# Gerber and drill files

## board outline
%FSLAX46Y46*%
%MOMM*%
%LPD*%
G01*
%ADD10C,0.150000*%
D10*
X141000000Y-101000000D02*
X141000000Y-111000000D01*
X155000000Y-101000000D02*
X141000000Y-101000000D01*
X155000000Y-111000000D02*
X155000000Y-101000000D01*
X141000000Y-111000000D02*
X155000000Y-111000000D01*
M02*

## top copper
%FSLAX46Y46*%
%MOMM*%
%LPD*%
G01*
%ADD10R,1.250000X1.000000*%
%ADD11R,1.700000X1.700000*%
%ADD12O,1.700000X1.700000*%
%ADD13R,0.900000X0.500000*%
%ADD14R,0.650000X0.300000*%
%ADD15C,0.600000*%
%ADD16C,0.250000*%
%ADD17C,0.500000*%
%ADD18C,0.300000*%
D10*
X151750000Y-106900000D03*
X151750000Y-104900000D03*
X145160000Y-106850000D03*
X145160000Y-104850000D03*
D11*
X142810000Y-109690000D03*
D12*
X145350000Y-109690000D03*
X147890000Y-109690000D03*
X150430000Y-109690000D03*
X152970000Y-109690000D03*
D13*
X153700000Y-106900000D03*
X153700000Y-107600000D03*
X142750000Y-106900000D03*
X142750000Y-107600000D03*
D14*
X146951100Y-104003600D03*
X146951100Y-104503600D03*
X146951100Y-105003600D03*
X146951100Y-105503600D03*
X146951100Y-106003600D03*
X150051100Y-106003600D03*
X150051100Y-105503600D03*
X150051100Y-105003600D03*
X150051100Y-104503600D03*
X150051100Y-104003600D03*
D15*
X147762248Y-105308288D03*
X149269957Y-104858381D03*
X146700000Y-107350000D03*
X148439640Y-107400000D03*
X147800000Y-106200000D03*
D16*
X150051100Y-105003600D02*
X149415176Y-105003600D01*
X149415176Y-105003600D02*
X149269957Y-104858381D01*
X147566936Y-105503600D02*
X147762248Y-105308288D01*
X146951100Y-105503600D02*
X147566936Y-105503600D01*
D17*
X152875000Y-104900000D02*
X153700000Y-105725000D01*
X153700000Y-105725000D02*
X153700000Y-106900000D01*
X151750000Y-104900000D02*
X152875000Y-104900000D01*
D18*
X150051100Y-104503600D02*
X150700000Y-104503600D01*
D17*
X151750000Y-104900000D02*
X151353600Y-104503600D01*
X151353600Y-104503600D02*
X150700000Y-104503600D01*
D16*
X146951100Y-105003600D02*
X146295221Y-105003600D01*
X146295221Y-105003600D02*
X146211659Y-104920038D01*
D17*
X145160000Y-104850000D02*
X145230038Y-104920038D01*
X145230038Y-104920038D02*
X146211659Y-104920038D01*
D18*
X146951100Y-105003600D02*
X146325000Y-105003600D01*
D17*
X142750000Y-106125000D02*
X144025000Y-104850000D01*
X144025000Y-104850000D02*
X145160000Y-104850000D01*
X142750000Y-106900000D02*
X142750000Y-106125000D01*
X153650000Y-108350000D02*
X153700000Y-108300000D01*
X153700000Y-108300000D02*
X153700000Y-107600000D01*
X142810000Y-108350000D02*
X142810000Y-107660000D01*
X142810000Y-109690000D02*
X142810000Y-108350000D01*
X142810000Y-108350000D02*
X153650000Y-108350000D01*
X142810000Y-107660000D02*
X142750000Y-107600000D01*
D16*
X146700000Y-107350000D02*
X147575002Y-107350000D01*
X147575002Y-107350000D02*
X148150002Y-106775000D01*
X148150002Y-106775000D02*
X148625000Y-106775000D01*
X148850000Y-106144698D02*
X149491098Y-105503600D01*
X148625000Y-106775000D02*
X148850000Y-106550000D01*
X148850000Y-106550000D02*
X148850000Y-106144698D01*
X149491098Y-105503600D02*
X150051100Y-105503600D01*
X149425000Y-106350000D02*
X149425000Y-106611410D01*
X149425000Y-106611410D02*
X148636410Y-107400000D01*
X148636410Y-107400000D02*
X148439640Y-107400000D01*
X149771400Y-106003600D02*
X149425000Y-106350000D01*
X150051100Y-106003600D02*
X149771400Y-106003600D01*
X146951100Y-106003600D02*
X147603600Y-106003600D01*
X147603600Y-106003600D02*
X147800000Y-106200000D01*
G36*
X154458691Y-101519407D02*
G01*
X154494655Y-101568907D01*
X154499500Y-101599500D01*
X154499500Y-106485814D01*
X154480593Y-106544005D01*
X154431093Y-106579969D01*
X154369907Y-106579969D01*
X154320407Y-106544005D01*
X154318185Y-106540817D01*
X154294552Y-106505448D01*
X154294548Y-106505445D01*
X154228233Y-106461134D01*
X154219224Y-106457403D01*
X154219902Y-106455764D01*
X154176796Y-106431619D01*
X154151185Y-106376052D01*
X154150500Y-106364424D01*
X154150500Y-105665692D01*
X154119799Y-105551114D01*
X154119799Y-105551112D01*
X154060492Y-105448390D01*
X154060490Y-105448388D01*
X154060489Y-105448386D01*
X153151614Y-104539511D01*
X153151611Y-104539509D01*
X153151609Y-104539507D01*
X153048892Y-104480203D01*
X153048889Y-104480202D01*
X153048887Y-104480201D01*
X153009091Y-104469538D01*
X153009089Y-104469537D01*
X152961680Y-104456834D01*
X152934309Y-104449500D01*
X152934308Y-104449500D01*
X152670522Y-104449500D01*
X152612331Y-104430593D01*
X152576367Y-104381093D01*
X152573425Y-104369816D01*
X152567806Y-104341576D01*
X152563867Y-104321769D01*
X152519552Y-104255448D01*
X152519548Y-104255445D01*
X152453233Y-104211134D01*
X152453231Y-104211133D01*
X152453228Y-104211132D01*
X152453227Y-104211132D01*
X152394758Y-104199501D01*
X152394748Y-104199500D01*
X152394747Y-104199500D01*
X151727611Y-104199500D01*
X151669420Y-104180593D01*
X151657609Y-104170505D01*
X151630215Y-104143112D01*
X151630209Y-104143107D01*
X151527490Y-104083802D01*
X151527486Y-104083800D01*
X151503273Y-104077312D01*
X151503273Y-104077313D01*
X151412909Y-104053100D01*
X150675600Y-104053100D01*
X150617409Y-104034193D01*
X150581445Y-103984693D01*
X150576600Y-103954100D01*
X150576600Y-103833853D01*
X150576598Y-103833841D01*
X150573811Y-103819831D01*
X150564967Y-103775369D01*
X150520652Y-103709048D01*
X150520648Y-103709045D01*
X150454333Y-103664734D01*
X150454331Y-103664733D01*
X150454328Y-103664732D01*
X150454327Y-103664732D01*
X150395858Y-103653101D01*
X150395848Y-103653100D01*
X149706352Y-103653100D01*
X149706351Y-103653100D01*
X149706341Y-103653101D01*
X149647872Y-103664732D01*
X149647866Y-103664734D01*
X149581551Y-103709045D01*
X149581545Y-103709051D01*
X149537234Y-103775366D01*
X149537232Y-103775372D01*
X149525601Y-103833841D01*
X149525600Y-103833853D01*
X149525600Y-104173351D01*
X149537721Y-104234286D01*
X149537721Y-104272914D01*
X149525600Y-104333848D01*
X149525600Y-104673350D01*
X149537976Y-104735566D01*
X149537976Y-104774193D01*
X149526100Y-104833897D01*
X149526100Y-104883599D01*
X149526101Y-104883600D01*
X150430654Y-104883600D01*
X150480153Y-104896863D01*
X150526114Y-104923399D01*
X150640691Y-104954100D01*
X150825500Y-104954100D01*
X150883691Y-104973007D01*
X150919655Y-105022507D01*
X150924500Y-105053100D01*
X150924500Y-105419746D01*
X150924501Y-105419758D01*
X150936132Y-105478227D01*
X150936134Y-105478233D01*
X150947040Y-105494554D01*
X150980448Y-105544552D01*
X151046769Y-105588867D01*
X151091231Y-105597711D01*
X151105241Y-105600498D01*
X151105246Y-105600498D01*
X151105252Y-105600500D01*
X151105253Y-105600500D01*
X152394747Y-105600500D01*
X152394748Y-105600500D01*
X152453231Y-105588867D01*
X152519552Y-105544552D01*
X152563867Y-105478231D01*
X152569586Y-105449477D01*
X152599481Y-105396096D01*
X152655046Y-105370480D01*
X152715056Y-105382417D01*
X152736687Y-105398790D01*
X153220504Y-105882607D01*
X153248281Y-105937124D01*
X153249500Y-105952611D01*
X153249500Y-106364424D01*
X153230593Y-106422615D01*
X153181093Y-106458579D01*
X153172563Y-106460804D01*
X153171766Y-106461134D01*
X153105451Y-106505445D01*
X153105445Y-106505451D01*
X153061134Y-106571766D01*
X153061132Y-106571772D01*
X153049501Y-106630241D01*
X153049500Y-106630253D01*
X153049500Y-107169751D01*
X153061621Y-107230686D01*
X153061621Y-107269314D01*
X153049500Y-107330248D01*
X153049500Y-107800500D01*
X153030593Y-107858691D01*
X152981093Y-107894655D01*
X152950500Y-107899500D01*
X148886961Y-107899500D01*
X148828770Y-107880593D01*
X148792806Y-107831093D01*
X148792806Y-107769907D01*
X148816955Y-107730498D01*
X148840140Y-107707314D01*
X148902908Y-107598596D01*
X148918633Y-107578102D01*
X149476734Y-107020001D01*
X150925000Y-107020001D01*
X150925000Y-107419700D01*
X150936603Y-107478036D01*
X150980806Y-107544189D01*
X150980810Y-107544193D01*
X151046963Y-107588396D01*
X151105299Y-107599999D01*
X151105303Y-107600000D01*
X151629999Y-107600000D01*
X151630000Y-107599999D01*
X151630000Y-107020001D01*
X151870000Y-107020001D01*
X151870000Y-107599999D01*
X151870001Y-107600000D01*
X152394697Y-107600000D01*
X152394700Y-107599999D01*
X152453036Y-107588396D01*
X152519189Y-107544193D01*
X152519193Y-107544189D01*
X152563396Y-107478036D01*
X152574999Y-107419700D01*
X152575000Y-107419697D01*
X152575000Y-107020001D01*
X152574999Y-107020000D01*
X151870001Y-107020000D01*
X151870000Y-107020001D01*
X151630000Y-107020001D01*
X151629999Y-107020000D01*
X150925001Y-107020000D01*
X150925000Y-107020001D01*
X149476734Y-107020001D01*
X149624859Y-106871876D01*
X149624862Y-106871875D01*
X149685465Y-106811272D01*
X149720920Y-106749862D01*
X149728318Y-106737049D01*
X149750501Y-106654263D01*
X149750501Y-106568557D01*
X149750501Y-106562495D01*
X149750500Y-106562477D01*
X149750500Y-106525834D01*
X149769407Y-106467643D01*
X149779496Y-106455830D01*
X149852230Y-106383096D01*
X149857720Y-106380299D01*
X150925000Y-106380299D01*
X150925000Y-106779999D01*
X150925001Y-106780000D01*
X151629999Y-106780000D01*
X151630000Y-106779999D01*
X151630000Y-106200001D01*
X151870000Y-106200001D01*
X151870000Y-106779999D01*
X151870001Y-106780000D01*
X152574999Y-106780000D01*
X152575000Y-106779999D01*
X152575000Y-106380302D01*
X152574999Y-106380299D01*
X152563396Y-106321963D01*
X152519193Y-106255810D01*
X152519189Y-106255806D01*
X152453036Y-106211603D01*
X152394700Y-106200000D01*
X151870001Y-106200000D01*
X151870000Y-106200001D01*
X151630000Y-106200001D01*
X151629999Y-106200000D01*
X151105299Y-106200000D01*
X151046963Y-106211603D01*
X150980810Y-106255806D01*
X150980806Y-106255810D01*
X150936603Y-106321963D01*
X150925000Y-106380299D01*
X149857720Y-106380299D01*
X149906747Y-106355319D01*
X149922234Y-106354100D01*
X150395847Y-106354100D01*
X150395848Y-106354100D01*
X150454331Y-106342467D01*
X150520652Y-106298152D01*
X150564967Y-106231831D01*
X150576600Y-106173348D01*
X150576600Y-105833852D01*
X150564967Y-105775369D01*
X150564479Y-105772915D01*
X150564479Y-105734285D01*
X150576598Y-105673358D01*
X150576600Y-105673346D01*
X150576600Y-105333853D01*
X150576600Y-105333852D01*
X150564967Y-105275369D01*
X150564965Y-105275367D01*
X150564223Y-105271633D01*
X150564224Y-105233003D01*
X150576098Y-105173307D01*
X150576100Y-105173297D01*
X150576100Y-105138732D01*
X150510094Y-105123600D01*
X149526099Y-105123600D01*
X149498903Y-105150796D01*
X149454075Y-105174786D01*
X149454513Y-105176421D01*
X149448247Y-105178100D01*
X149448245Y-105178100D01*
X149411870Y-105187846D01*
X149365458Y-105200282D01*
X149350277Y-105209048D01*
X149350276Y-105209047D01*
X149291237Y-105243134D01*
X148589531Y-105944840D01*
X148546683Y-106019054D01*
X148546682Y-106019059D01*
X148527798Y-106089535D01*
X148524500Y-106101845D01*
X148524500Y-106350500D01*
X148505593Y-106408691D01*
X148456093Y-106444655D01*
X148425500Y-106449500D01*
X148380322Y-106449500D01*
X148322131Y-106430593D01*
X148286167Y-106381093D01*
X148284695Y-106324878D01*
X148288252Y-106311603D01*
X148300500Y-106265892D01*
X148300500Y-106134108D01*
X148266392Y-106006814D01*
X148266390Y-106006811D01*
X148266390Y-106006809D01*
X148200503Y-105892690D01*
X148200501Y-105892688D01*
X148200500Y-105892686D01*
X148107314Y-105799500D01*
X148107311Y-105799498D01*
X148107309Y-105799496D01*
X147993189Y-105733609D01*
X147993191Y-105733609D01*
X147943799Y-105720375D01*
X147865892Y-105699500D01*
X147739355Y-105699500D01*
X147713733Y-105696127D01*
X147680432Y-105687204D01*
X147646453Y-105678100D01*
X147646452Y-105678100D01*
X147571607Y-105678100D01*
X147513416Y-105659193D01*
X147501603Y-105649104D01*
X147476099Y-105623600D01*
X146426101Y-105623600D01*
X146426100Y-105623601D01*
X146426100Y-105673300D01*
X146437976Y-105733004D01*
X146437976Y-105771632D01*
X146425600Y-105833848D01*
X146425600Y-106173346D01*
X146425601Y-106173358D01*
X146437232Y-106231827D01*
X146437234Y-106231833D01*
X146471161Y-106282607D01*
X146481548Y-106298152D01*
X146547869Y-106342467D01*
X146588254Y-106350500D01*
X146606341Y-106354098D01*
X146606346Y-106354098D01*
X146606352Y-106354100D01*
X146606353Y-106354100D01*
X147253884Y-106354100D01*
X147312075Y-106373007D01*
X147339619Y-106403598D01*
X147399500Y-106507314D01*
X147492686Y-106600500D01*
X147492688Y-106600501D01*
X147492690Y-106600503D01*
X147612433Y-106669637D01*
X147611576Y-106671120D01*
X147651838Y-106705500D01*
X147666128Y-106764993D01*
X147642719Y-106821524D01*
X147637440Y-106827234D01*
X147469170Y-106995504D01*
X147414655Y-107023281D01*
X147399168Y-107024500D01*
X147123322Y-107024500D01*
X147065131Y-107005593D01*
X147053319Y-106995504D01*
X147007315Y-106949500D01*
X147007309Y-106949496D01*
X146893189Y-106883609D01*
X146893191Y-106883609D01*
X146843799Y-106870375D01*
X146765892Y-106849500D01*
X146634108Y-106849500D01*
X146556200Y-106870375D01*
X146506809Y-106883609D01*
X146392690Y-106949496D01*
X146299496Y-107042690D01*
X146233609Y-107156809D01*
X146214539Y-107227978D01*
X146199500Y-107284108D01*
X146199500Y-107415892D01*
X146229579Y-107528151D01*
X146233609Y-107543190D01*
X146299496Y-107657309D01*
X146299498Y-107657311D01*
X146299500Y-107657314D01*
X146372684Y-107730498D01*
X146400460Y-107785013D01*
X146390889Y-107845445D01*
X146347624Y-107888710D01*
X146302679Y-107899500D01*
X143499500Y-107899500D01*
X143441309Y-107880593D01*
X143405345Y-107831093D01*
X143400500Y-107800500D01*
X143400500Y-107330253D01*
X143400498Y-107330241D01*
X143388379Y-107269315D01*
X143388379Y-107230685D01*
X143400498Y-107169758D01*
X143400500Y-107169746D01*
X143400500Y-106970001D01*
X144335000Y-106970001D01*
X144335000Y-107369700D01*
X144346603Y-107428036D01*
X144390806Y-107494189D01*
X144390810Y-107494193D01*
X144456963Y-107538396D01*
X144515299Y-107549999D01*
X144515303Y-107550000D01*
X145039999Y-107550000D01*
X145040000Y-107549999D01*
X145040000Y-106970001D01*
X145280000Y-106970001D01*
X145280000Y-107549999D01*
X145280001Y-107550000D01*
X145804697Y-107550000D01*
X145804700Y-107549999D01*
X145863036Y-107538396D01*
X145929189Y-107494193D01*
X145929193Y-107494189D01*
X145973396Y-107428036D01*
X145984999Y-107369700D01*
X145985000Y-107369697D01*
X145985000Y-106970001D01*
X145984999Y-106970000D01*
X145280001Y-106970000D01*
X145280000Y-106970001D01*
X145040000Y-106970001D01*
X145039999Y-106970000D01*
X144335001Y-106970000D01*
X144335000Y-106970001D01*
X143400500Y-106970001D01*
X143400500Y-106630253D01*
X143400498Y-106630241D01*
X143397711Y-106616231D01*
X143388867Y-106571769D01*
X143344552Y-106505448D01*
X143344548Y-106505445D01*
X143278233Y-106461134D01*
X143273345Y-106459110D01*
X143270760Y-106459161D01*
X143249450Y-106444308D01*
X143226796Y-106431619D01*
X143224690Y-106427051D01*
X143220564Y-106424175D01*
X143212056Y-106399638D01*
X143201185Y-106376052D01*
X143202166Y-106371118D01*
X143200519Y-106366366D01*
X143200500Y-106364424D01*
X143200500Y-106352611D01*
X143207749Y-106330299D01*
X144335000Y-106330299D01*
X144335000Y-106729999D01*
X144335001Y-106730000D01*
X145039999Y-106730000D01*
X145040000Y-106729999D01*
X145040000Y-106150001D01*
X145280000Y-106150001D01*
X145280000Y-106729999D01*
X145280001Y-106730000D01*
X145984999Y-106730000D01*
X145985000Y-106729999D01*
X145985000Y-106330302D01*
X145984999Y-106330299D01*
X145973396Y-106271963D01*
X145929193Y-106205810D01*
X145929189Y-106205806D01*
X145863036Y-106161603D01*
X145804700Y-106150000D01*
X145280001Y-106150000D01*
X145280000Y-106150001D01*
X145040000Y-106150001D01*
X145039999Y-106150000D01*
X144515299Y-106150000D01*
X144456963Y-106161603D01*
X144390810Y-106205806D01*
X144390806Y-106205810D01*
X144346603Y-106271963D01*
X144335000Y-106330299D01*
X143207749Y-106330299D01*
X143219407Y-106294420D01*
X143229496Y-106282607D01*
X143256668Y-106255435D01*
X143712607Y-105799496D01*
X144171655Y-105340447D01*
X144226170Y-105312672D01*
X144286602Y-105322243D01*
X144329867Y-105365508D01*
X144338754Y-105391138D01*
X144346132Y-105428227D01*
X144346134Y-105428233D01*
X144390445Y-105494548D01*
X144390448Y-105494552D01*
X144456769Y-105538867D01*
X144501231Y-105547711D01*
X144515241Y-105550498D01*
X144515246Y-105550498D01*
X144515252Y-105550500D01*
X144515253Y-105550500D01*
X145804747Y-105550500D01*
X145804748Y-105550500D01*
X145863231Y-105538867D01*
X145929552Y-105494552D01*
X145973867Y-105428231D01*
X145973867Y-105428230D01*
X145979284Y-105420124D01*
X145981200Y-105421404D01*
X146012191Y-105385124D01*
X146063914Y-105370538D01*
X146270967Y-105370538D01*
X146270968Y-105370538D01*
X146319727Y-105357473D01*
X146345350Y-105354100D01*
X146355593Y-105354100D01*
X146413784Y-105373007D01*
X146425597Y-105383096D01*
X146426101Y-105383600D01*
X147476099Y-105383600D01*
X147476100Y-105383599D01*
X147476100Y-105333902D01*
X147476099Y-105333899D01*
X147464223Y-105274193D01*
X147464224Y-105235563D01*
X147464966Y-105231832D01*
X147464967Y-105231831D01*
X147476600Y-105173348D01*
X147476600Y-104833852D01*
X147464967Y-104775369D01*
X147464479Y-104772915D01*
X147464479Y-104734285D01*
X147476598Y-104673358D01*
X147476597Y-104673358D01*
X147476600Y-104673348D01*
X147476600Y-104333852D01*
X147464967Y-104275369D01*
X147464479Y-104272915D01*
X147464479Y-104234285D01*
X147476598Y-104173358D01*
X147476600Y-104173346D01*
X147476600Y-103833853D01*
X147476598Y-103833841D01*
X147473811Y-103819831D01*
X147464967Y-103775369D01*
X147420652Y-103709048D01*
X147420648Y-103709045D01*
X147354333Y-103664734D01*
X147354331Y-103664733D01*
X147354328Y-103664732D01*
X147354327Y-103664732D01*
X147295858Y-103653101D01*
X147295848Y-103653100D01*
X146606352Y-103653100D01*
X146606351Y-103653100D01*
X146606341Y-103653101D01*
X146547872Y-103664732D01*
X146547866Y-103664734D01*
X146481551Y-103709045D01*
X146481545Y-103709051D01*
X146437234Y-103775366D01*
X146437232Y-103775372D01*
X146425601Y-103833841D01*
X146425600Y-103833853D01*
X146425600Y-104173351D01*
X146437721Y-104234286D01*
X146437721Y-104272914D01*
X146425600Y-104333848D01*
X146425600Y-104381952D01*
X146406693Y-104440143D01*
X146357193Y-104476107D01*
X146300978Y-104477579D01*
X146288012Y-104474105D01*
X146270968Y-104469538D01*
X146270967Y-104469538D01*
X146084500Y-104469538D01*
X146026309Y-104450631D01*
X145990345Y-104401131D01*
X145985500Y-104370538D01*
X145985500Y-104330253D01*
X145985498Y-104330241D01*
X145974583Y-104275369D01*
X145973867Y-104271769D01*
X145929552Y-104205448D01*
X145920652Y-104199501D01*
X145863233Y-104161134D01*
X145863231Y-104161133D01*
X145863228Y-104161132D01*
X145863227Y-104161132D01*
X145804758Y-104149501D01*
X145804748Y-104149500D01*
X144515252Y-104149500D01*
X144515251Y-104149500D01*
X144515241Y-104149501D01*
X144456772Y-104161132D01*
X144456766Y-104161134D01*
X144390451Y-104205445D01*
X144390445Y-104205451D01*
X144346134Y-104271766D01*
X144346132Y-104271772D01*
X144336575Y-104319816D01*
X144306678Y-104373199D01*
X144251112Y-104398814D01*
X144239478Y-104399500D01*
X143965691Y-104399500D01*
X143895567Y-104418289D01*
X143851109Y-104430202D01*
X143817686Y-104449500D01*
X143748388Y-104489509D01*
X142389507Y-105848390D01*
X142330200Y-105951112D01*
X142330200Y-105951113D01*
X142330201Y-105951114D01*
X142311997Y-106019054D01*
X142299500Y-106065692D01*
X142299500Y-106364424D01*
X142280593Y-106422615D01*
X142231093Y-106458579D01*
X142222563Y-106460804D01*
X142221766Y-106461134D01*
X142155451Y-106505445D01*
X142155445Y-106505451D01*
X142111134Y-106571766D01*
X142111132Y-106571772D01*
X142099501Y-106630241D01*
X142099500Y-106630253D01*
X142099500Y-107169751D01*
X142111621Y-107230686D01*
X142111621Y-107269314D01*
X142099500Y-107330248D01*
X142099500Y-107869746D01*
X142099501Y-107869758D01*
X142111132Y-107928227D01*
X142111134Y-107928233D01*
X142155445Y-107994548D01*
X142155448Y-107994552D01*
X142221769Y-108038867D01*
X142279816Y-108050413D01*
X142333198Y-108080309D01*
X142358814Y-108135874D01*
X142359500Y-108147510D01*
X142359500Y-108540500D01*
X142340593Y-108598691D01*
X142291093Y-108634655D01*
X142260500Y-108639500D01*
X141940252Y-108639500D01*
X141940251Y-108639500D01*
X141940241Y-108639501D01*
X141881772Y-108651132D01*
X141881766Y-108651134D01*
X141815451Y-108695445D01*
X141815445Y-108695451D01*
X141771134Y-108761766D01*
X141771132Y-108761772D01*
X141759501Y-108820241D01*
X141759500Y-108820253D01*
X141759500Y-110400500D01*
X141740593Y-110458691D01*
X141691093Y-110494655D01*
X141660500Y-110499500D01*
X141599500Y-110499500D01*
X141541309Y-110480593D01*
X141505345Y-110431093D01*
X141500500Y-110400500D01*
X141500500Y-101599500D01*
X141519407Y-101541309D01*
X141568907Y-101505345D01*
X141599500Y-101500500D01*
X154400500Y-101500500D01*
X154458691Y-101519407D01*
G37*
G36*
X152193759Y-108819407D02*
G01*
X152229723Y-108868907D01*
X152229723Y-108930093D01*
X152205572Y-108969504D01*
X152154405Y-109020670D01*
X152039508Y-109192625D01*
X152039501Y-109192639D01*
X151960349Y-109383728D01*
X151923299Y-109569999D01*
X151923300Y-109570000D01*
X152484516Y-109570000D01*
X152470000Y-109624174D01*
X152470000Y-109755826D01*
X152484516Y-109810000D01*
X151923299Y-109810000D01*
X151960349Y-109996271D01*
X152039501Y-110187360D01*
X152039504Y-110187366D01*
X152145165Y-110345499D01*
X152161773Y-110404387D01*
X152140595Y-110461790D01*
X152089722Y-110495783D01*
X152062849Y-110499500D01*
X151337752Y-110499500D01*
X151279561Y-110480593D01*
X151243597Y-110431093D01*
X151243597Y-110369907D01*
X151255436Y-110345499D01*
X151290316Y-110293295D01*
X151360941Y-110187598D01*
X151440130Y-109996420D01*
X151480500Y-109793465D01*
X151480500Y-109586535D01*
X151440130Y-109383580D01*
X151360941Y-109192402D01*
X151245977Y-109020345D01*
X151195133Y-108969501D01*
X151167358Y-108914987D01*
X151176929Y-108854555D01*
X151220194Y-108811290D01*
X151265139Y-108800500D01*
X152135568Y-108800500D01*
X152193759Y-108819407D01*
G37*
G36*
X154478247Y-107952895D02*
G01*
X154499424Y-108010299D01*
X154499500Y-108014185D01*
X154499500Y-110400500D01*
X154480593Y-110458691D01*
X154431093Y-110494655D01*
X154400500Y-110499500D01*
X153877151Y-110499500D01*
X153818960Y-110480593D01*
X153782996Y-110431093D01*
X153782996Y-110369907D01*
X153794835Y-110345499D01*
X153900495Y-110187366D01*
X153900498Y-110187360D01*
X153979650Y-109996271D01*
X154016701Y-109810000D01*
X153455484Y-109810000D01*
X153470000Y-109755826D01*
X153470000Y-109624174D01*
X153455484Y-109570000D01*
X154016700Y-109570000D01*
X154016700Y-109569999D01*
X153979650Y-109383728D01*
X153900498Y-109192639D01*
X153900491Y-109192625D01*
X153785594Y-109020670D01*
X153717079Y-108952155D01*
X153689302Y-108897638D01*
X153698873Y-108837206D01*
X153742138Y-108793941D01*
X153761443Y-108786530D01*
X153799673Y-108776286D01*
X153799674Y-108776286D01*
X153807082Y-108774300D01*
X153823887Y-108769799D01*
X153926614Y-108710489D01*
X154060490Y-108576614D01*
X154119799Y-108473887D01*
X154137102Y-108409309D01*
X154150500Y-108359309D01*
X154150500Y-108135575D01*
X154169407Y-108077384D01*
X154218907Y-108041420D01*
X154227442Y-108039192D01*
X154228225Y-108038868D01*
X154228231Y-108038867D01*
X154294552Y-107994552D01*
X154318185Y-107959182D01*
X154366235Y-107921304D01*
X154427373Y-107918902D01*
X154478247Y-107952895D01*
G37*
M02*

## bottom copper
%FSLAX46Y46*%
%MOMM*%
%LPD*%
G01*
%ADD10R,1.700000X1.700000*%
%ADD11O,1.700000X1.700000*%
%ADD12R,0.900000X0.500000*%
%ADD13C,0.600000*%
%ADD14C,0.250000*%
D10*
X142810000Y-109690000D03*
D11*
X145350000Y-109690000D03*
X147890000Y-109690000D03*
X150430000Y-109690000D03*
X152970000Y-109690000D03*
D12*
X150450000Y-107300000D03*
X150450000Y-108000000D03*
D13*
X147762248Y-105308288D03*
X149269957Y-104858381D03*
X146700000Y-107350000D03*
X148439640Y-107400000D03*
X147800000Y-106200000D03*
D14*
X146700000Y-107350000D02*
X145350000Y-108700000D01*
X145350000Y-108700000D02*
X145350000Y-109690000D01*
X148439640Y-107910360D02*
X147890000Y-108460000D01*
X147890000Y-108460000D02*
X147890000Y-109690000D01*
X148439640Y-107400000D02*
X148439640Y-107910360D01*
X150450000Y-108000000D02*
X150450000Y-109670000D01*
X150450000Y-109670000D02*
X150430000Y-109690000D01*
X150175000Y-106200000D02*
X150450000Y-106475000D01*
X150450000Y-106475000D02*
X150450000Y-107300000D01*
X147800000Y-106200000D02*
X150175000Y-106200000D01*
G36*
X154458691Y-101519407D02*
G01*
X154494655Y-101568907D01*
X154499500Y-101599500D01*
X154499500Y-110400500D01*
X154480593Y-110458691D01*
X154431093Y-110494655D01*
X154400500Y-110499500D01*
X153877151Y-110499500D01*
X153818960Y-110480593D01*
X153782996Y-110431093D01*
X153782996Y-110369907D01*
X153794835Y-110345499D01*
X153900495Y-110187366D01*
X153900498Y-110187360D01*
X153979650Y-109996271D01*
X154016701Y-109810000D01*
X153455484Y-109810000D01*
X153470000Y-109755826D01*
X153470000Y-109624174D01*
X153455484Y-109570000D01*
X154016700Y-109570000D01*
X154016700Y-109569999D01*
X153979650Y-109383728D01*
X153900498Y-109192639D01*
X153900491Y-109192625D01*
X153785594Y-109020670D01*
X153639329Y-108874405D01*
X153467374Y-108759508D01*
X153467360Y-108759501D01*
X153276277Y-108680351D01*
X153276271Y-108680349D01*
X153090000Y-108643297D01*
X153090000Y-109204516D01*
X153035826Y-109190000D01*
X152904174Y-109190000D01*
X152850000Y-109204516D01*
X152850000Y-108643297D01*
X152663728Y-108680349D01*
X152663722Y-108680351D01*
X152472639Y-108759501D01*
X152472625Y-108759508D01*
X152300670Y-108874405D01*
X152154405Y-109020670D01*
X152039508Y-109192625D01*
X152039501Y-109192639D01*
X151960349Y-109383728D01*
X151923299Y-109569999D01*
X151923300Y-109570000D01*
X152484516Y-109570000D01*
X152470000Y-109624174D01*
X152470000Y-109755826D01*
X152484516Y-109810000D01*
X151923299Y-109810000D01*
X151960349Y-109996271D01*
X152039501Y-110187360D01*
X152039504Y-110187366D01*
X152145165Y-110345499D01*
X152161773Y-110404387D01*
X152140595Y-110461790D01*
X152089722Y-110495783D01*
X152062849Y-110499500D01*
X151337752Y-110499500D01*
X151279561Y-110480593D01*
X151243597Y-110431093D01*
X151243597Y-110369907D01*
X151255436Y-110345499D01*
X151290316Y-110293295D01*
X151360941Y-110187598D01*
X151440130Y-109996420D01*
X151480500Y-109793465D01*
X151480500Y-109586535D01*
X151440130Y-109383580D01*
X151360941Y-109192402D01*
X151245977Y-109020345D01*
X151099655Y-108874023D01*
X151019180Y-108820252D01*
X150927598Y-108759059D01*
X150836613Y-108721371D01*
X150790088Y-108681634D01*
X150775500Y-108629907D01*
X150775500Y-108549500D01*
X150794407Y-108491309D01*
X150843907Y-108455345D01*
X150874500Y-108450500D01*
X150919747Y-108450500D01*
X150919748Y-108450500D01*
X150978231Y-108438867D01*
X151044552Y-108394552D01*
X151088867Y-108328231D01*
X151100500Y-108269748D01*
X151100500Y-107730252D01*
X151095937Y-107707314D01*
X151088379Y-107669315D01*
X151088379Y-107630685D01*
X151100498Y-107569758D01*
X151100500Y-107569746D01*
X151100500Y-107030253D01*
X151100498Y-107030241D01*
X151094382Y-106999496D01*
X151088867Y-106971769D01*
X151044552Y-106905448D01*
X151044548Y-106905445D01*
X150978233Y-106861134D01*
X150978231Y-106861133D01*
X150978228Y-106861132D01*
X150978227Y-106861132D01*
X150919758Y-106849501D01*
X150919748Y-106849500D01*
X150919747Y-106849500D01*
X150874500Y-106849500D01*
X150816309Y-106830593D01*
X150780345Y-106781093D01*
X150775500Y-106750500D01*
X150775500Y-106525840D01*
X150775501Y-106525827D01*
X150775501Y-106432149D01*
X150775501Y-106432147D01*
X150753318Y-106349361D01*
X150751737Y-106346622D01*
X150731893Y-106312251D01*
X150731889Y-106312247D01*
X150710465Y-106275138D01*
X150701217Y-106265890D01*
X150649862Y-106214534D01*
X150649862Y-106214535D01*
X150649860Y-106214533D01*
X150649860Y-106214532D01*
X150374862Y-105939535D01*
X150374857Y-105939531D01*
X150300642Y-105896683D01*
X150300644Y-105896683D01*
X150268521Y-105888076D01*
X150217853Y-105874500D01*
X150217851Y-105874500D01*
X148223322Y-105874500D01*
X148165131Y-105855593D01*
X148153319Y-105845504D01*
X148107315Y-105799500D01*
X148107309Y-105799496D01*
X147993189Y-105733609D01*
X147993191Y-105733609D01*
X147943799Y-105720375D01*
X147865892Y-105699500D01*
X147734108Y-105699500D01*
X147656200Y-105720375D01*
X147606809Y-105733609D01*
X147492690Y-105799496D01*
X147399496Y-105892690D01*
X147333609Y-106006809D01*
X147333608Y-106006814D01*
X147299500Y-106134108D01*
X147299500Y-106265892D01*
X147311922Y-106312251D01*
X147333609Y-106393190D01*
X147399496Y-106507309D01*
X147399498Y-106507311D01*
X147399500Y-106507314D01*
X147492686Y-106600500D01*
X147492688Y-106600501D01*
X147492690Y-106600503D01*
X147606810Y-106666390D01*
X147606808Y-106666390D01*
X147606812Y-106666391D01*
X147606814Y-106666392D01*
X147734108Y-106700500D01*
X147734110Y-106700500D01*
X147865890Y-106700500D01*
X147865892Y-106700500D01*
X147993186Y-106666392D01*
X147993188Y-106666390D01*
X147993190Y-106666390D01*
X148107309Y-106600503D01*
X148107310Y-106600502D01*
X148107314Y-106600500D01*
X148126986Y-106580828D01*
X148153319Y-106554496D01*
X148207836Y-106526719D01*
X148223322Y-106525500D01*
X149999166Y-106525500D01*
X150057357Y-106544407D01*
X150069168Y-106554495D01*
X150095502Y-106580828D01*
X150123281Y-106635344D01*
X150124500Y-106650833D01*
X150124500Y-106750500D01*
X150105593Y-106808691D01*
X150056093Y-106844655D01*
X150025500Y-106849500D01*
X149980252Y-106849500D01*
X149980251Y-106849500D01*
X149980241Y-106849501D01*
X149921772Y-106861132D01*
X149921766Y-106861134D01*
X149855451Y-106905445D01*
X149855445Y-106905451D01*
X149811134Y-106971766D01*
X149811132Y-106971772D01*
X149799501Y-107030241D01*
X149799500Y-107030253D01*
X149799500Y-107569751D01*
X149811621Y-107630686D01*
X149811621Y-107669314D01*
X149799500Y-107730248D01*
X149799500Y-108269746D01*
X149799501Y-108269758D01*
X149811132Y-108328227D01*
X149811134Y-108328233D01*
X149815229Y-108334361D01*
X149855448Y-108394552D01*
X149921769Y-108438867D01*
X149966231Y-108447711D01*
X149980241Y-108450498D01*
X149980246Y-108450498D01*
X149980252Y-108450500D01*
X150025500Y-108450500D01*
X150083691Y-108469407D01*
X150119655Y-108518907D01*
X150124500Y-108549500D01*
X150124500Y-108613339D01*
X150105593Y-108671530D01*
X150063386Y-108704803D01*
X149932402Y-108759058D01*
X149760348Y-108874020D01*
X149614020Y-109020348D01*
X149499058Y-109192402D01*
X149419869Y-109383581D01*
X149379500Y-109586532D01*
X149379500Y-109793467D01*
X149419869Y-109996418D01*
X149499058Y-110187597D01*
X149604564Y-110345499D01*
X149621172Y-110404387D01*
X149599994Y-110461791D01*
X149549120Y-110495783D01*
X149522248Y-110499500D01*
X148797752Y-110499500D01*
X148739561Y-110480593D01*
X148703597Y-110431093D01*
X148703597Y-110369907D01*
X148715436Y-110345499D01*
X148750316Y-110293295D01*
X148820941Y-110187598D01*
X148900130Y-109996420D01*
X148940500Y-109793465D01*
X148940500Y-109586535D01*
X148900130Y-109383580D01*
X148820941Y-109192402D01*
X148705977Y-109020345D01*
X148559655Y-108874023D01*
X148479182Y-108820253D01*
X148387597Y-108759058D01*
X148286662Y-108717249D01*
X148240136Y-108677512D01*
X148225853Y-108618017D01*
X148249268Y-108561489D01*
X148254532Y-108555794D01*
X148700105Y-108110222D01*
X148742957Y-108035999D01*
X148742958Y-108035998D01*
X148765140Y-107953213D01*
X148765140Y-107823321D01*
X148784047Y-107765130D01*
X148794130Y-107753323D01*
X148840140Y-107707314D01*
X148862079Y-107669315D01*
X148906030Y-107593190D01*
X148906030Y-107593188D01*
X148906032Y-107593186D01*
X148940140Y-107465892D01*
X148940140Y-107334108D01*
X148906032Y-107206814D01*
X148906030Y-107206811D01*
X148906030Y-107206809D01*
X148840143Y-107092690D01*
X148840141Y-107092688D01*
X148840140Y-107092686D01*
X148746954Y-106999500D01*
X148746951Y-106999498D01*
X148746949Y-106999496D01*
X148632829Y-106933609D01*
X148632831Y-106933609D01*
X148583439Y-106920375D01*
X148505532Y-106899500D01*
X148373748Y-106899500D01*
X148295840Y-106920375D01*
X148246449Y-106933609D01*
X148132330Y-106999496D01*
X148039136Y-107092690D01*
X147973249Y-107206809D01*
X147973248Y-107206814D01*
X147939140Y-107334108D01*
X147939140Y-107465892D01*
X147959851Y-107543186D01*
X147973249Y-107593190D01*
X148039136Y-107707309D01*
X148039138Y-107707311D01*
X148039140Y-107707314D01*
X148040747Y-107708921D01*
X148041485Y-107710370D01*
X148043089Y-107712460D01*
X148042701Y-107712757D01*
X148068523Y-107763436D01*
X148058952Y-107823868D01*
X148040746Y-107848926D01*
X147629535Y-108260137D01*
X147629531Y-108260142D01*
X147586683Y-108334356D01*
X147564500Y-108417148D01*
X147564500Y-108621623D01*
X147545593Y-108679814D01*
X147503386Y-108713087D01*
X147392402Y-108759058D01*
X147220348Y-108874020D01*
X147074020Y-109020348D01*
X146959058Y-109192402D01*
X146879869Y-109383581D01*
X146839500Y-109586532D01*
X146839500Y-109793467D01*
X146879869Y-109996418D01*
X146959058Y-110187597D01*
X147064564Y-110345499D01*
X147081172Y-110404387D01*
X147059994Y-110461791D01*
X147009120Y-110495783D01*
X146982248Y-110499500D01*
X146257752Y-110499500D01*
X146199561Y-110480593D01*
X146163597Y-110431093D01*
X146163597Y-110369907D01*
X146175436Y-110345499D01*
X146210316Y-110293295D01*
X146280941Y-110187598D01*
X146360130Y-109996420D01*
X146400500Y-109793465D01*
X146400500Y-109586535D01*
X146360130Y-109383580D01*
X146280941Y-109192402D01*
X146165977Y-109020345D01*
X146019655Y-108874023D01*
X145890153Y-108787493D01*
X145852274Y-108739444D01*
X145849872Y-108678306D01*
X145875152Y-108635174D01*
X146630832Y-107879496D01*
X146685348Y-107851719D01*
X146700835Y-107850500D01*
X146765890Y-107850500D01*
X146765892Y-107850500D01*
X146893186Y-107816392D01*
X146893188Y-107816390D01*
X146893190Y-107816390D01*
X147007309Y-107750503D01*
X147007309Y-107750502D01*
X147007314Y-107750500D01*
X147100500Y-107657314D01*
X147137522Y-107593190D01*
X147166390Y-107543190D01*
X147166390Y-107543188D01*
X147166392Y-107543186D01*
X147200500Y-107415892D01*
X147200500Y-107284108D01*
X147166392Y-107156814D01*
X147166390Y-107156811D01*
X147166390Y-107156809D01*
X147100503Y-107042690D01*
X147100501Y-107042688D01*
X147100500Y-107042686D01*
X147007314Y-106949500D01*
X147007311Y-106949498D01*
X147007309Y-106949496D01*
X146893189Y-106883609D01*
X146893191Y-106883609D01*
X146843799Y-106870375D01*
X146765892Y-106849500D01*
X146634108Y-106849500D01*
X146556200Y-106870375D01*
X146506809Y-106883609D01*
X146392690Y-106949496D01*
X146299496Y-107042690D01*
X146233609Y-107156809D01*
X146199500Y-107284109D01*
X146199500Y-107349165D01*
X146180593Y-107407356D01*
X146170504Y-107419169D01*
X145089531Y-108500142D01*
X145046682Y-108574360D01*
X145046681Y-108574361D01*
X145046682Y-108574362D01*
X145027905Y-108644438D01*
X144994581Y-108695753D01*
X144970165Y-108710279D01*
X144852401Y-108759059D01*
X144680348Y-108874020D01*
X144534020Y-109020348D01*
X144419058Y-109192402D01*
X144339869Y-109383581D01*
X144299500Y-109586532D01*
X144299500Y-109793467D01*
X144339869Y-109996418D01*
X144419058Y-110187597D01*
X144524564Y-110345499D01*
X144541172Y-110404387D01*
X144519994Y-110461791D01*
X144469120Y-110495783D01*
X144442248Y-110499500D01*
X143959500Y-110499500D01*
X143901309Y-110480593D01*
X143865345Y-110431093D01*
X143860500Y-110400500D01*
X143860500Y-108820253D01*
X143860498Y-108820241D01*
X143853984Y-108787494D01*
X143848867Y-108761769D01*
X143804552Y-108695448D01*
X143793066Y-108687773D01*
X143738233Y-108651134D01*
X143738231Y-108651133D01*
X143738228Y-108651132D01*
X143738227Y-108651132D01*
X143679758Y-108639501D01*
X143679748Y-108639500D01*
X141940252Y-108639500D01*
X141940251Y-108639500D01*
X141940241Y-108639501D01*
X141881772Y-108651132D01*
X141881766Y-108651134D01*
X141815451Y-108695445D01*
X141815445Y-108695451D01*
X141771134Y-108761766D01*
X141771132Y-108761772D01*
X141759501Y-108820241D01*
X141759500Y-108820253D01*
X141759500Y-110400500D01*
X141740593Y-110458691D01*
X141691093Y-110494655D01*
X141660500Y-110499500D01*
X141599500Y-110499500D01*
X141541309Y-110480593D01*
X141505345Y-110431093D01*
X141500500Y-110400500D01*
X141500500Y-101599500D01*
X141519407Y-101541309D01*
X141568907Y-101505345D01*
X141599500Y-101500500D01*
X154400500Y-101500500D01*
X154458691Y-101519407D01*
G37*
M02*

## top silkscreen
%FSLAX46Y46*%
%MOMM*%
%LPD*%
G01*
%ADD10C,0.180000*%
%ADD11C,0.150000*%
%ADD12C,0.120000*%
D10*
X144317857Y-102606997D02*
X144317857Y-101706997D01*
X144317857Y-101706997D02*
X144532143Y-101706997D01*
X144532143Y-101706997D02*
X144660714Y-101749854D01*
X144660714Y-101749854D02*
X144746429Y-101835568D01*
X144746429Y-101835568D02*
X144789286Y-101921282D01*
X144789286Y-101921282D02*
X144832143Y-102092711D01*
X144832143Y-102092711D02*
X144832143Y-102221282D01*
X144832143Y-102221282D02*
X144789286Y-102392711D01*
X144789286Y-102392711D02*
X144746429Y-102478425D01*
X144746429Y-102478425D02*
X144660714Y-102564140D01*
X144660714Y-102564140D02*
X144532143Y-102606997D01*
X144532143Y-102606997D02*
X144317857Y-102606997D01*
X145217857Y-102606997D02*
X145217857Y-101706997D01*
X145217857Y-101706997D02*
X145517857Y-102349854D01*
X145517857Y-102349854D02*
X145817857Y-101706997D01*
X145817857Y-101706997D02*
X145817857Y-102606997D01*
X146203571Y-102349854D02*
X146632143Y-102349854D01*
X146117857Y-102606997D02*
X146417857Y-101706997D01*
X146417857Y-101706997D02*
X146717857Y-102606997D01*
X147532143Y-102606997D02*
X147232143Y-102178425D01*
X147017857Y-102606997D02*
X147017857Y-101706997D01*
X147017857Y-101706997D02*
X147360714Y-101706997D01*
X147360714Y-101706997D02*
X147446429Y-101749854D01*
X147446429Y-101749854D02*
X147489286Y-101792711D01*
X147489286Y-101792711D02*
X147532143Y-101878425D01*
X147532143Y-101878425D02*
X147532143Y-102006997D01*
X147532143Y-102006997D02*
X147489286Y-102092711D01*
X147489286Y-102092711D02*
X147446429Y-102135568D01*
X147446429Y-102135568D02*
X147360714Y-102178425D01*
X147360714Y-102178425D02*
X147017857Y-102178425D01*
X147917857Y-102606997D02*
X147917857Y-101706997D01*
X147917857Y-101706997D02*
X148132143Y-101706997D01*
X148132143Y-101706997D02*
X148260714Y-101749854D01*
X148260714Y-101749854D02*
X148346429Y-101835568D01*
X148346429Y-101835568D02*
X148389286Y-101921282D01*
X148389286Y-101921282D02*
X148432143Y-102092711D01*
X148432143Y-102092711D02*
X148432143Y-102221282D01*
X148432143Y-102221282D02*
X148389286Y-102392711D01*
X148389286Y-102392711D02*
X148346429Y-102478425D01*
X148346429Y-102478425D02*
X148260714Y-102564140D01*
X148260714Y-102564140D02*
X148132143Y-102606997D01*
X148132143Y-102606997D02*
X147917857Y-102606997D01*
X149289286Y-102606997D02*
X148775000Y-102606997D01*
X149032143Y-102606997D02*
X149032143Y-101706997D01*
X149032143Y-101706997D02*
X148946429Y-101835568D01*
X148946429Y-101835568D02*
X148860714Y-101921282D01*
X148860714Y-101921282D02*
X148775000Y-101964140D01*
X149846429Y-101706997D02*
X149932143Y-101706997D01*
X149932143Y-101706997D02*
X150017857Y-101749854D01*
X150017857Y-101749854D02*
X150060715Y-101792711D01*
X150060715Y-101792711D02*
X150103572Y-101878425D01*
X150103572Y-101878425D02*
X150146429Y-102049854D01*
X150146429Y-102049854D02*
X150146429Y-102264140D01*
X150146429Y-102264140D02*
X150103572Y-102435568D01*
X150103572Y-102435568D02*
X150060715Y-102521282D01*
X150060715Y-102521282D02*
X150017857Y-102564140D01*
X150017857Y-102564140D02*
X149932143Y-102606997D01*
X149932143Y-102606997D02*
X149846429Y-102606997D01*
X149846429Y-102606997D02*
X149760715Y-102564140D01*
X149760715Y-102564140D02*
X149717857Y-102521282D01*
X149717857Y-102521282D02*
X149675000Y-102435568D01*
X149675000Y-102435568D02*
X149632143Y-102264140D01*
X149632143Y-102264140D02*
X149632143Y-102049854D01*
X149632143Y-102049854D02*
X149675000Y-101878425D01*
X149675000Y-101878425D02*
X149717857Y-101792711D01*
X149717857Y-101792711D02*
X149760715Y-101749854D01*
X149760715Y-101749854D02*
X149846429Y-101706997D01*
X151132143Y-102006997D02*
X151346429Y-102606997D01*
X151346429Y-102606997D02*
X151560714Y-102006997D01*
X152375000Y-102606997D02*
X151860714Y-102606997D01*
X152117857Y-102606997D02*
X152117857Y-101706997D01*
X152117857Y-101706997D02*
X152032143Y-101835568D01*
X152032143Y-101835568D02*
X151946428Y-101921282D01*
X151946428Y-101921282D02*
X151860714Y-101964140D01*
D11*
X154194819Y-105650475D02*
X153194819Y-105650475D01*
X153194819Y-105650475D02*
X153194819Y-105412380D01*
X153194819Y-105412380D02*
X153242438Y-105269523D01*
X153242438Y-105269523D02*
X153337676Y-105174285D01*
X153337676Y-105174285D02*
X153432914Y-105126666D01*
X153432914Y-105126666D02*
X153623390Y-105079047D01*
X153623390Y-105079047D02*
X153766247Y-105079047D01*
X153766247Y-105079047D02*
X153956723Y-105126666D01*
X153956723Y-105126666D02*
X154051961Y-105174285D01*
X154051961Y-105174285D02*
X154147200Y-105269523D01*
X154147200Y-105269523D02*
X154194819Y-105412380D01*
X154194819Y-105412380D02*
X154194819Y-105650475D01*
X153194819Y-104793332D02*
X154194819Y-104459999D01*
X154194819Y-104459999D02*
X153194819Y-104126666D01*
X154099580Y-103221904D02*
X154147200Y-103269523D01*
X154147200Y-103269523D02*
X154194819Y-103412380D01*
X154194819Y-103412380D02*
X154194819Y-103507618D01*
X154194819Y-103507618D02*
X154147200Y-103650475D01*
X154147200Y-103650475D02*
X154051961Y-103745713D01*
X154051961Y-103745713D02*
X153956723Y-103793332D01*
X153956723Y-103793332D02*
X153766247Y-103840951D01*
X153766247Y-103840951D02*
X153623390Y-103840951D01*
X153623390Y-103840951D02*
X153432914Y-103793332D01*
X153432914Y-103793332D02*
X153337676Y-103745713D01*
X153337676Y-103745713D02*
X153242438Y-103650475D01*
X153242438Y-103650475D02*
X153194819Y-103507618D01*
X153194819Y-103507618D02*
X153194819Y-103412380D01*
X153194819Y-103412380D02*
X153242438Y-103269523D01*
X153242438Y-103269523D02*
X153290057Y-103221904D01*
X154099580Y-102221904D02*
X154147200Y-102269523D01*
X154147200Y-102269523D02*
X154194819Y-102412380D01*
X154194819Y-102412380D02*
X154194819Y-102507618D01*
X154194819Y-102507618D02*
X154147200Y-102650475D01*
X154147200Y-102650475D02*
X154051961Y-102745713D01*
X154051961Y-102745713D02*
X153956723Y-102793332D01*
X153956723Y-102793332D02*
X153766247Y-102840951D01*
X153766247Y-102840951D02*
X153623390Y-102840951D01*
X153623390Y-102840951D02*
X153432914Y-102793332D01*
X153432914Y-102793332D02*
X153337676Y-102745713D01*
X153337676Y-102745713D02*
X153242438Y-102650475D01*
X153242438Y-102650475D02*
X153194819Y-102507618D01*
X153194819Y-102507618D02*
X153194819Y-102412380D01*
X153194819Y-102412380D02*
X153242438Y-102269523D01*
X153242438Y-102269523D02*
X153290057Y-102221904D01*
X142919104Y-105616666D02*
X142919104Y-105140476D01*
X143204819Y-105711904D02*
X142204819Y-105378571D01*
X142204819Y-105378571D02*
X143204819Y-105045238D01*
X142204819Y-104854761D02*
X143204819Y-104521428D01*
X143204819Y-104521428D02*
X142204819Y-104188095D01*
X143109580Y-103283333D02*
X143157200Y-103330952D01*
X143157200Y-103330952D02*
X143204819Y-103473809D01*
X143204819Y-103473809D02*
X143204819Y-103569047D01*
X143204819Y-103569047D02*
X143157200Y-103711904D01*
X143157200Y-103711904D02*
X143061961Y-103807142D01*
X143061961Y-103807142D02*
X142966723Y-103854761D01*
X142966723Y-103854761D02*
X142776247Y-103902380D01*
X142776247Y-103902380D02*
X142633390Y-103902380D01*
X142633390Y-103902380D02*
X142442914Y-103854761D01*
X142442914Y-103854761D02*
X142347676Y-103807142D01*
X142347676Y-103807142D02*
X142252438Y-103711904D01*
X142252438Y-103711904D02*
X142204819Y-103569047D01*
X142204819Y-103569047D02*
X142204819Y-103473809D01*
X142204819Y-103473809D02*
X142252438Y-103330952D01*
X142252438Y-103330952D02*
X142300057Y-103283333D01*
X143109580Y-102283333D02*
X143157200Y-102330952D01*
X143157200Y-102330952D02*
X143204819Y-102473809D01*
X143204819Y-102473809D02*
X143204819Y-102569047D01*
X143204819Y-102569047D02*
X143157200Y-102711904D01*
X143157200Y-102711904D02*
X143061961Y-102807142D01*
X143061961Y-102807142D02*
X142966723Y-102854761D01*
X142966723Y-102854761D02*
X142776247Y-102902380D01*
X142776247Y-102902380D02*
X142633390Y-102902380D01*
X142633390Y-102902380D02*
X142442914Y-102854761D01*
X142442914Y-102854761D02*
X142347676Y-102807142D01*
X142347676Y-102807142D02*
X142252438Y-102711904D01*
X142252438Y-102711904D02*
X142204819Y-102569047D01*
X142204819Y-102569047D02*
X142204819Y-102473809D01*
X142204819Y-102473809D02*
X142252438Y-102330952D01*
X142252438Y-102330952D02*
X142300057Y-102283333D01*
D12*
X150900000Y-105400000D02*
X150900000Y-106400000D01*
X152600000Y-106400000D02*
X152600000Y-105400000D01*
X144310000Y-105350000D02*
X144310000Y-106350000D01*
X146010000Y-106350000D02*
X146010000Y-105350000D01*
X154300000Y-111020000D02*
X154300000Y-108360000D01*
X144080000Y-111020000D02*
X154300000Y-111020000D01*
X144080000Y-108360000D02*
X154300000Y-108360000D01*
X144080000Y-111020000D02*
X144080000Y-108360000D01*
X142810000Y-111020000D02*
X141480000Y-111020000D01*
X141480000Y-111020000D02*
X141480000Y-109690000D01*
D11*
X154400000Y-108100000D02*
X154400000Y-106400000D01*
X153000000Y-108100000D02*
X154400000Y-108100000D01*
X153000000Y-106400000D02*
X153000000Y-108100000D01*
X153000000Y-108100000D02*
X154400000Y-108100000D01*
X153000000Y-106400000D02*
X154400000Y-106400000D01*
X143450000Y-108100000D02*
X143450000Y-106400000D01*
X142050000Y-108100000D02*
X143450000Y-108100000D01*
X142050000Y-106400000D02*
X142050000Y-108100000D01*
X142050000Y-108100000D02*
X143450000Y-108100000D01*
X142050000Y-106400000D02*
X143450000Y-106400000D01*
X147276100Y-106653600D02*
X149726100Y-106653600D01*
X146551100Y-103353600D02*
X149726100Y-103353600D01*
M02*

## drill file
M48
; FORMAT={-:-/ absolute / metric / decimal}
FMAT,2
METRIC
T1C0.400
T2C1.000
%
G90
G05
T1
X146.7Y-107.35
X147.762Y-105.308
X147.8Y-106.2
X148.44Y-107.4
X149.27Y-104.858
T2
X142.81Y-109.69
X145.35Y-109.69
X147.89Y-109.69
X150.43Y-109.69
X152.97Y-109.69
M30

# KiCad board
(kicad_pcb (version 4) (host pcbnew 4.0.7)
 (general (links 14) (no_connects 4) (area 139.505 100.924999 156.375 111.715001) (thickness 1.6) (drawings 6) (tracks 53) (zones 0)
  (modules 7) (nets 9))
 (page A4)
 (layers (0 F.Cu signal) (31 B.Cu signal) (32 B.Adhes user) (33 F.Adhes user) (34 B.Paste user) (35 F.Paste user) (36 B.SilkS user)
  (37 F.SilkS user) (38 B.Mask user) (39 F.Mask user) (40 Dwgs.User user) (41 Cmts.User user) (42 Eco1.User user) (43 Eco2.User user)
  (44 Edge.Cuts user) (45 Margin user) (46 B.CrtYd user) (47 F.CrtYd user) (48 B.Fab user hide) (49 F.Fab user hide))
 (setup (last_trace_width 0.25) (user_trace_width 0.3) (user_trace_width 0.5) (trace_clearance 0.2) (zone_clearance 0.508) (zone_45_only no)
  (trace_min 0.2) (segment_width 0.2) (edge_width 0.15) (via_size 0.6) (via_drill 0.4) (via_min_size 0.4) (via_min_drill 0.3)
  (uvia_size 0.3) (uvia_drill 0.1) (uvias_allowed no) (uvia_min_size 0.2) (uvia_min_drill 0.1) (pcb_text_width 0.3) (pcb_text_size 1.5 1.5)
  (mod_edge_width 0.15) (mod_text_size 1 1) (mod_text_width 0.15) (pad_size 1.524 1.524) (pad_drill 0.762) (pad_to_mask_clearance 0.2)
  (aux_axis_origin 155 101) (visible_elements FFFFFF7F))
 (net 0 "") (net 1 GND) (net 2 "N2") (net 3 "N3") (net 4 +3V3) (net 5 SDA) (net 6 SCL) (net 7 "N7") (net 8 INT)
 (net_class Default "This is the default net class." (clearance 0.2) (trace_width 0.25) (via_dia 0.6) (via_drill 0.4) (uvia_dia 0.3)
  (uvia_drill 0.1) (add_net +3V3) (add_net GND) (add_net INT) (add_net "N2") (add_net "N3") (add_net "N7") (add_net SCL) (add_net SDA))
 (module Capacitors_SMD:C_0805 (layer F.Cu) (at 151.75 105.9 90)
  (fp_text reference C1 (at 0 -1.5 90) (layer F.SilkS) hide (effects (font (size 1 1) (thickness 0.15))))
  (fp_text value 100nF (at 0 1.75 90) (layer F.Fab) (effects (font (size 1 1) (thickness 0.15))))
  (fp_line (start 0.5 -0.85) (end -0.5 -0.85) (layer F.SilkS) (width 0.12))
  (fp_line (start -0.5 0.85) (end 0.5 0.85) (layer F.SilkS) (width 0.12))
  (pad 1 smd rect (at -1 0 90) (size 1 1.25) (layers F.Cu F.Paste F.Mask) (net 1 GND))
  (pad 2 smd rect (at 1 0 90) (size 1 1.25) (layers F.Cu F.Paste F.Mask) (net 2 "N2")))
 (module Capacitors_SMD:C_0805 (layer F.Cu) (at 145.16 105.85 90)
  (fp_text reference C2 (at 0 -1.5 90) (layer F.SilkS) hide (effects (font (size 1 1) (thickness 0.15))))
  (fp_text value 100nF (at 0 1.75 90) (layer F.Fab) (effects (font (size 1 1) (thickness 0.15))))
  (fp_line (start 0.5 -0.85) (end -0.5 -0.85) (layer F.SilkS) (width 0.12))
  (fp_line (start -0.5 0.85) (end 0.5 0.85) (layer F.SilkS) (width 0.12))
  (pad 1 smd rect (at -1 0 90) (size 1 1.25) (layers F.Cu F.Paste F.Mask) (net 1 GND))
  (pad 2 smd rect (at 1 0 90) (size 1 1.25) (layers F.Cu F.Paste F.Mask) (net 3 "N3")))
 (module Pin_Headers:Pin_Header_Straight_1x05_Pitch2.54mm (layer F.Cu) (at 142.81 109.69 90)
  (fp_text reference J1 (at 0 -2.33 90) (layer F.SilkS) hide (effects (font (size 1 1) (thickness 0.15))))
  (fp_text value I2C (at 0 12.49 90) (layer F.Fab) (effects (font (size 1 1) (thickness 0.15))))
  (fp_line (start -1.33 11.49) (end 1.33 11.49) (layer F.SilkS) (width 0.12))
  (fp_line (start -1.33 1.27) (end -1.33 11.49) (layer F.SilkS) (width 0.12))
  (fp_line (start 1.33 1.27) (end 1.33 11.49) (layer F.SilkS) (width 0.12))
  (fp_line (start -1.33 1.27) (end 1.33 1.27) (layer F.SilkS) (width 0.12))
  (fp_line (start -1.33 0) (end -1.33 -1.33) (layer F.SilkS) (width 0.12))
  (fp_line (start -1.33 -1.33) (end 0 -1.33) (layer F.SilkS) (width 0.12))
  (pad 1 thru_hole rect (at 0 0 90) (size 1.7 1.7) (drill 1) (layers *.Cu *.Mask) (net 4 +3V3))
  (pad 2 thru_hole oval (at 0 2.54 90) (size 1.7 1.7) (drill 1) (layers *.Cu *.Mask) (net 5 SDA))
  (pad 3 thru_hole oval (at 0 5.08 90) (size 1.7 1.7) (drill 1) (layers *.Cu *.Mask) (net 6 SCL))
  (pad 4 thru_hole oval (at 0 7.62 90) (size 1.7 1.7) (drill 1) (layers *.Cu *.Mask) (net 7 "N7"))
  (pad 5 thru_hole oval (at 0 10.16 90) (size 1.7 1.7) (drill 1) (layers *.Cu *.Mask) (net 1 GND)))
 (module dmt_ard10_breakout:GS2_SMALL (layer F.Cu) (at 153.7 107.6)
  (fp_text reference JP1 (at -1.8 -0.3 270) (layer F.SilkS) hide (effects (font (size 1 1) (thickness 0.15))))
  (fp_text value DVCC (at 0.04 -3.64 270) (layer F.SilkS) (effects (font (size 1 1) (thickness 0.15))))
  (fp_line (start 0.7 0.5) (end 0.7 -1.2) (layer F.SilkS) (width 0.15))
  (fp_line (start -0.7 0.5) (end 0.7 0.5) (layer F.SilkS) (width 0.15))
  (fp_line (start -0.7 -1.2) (end -0.7 0.5) (layer F.SilkS) (width 0.15))
  (fp_line (start -0.7 0.5) (end 0.7 0.5) (layer F.SilkS) (width 0.15))
  (fp_line (start -0.7 -1.2) (end 0.7 -1.2) (layer F.SilkS) (width 0.15))
  (pad 1 smd rect (at 0 -0.7) (size 0.9 0.5) (layers F.Cu F.Paste F.Mask) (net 2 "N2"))
  (pad 2 smd rect (at 0 0) (size 0.9 0.5) (layers F.Cu F.Paste F.Mask) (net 4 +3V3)))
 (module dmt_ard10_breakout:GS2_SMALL (layer B.Cu) (at 150.45 108 180)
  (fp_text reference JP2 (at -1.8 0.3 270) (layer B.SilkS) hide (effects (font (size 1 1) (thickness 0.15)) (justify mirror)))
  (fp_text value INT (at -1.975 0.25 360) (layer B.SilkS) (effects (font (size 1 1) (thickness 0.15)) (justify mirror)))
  (pad 1 smd rect (at 0 0.7 180) (size 0.9 0.5) (layers B.Cu B.Paste B.Mask) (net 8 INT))
  (pad 2 smd rect (at 0 0 180) (size 0.9 0.5) (layers B.Cu B.Paste B.Mask) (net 7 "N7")))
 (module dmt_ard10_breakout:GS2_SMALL (layer F.Cu) (at 142.75 107.6)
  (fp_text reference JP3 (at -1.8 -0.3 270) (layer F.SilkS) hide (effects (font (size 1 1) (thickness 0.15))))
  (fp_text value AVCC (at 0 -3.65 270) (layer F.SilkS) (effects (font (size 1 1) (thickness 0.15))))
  (fp_line (start 0.7 0.5) (end 0.7 -1.2) (layer F.SilkS) (width 0.15))
  (fp_line (start -0.7 0.5) (end 0.7 0.5) (layer F.SilkS) (width 0.15))
  (fp_line (start -0.7 -1.2) (end -0.7 0.5) (layer F.SilkS) (width 0.15))
  (fp_line (start -0.7 0.5) (end 0.7 0.5) (layer F.SilkS) (width 0.15))
  (fp_line (start -0.7 -1.2) (end 0.7 -1.2) (layer F.SilkS) (width 0.15))
  (pad 1 smd rect (at 0 -0.7) (size 0.9 0.5) (layers F.Cu F.Paste F.Mask) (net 3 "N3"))
  (pad 2 smd rect (at 0 0) (size 0.9 0.5) (layers F.Cu F.Paste F.Mask) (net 4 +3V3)))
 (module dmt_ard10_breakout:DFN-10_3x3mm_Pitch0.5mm (layer F.Cu) (at 148.5011 105.0036)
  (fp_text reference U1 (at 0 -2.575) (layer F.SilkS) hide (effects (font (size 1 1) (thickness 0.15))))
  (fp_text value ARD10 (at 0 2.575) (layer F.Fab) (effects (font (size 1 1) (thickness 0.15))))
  (fp_line (start -1.225 1.65) (end 1.225 1.65) (layer F.SilkS) (width 0.15))
  (fp_line (start -1.95 -1.65) (end 1.225 -1.65) (layer F.SilkS) (width 0.15))
  (pad 1 smd rect (at -1.55 -1) (size 0.65 0.3) (layers F.Cu F.Paste F.Mask))
  (pad 2 smd rect (at -1.55 -0.5) (size 0.65 0.3) (layers F.Cu F.Paste F.Mask))
  (pad 3 smd rect (at -1.55 0) (size 0.65 0.3) (layers F.Cu F.Paste F.Mask) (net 3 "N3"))
  (pad 4 smd rect (at -1.55 0.5) (size 0.65 0.3) (layers F.Cu F.Paste F.Mask) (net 1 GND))
  (pad 5 smd rect (at -1.55 1) (size 0.65 0.3) (layers F.Cu F.Paste F.Mask) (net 8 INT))
  (pad 6 smd rect (at 1.55 1) (size 0.65 0.3) (layers F.Cu F.Paste F.Mask) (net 6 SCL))
  (pad 7 smd rect (at 1.55 0.5) (size 0.65 0.3) (layers F.Cu F.Paste F.Mask) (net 5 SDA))
  (pad 8 smd rect (at 1.55 0) (size 0.65 0.3) (layers F.Cu F.Paste F.Mask) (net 1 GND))
  (pad 9 smd rect (at 1.55 -0.5) (size 0.65 0.3) (layers F.Cu F.Paste F.Mask) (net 2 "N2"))
  (pad 10 smd rect (at 1.55 -1) (size 0.65 0.3) (layers F.Cu F.Paste F.Mask)))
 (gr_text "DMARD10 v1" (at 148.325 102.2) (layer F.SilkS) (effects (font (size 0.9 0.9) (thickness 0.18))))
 (gr_line (start 141 101) (end 141 111) (layer Edge.Cuts) (width 0.15))
 (gr_line (start 155 101) (end 141 101) (layer Edge.Cuts) (width 0.15))
 (gr_line (start 155 111) (end 155 101) (layer Edge.Cuts) (width 0.15))
 (gr_line (start 141 111) (end 155 111) (layer Edge.Cuts) (width 0.15))
 (segment (start 150.0511 105.0036) (end 149.415176 105.0036) (width 0.25) (layer F.Cu) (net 1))
 (segment (start 149.415176 105.0036) (end 149.269957 104.858381) (width 0.25) (layer F.Cu) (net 1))
 (segment (start 147.566936 105.5036) (end 147.762248 105.308288) (width 0.25) (layer F.Cu) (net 1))
 (segment (start 146.9511 105.5036) (end 147.566936 105.5036) (width 0.25) (layer F.Cu) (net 1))
 (via (at 147.762248 105.308288) (size 0.6) (drill 0.4) (layers F.Cu B.Cu) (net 1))
 (via (at 149.269957 104.858381) (size 0.6) (drill 0.4) (layers F.Cu B.Cu) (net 1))
 (segment (start 152.875 104.9) (end 153.7 105.725) (width 0.5) (layer F.Cu) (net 2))
 (segment (start 153.7 105.725) (end 153.7 106.9) (width 0.5) (layer F.Cu) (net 2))
 (segment (start 151.75 104.9) (end 152.875 104.9) (width 0.5) (layer F.Cu) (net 2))
 (segment (start 150.0511 104.5036) (end 150.7 104.5036) (width 0.3) (layer F.Cu) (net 2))
 (segment (start 151.75 104.9) (end 151.3536 104.5036) (width 0.5) (layer F.Cu) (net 2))
 (segment (start 151.3536 104.5036) (end 150.7 104.5036) (width 0.5) (layer F.Cu) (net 2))
 (segment (start 146.9511 105.0036) (end 146.295221 105.0036) (width 0.25) (layer F.Cu) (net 3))
 (segment (start 146.295221 105.0036) (end 146.211659 104.920038) (width 0.25) (layer F.Cu) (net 3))
 (segment (start 145.16 104.85) (end 145.230038 104.920038) (width 0.5) (layer F.Cu) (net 3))
 (segment (start 145.230038 104.920038) (end 146.211659 104.920038) (width 0.5) (layer F.Cu) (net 3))
 (segment (start 146.9511 105.0036) (end 146.325 105.0036) (width 0.3) (layer F.Cu) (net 3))
 (segment (start 142.75 106.125) (end 144.025 104.85) (width 0.5) (layer F.Cu) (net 3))
 (segment (start 144.025 104.85) (end 145.16 104.85) (width 0.5) (layer F.Cu) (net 3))
 (segment (start 142.75 106.9) (end 142.75 106.125) (width 0.5) (layer F.Cu) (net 3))
 (segment (start 153.65 108.35) (end 153.7 108.3) (width 0.5) (layer F.Cu) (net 4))
 (segment (start 153.7 108.3) (end 153.7 107.6) (width 0.5) (layer F.Cu) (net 4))
 (segment (start 142.81 108.35) (end 142.81 107.66) (width 0.5) (layer F.Cu) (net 4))
 (segment (start 142.81 109.69) (end 142.81 108.35) (width 0.5) (layer F.Cu) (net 4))
 (segment (start 142.81 108.35) (end 153.65 108.35) (width 0.5) (layer F.Cu) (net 4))
 (segment (start 142.81 107.66) (end 142.75 107.6) (width 0.5) (layer F.Cu) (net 4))
 (segment (start 146.7 107.35) (end 147.575002 107.35) (width 0.25) (layer F.Cu) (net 5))
 (segment (start 147.575002 107.35) (end 148.150002 106.775) (width 0.25) (layer F.Cu) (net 5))
 (segment (start 148.150002 106.775) (end 148.625 106.775) (width 0.25) (layer F.Cu) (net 5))
 (segment (start 148.85 106.144698) (end 149.491098 105.5036) (width 0.25) (layer F.Cu) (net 5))
 (segment (start 148.625 106.775) (end 148.85 106.55) (width 0.25) (layer F.Cu) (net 5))
 (segment (start 148.85 106.55) (end 148.85 106.144698) (width 0.25) (layer F.Cu) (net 5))
 (segment (start 149.491098 105.5036) (end 150.0511 105.5036) (width 0.25) (layer F.Cu) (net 5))
 (segment (start 146.7 107.35) (end 145.35 108.7) (width 0.25) (layer B.Cu) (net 5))
 (segment (start 145.35 108.7) (end 145.35 109.69) (width 0.25) (layer B.Cu) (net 5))
 (via (at 146.7 107.35) (size 0.6) (drill 0.4) (layers F.Cu B.Cu) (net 5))
 (segment (start 148.43964 107.91036) (end 147.89 108.46) (width 0.25) (layer B.Cu) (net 6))
 (segment (start 147.89 108.46) (end 147.89 109.69) (width 0.25) (layer B.Cu) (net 6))
 (segment (start 148.43964 107.4) (end 148.43964 107.91036) (width 0.25) (layer B.Cu) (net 6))
 (segment (start 149.425 106.35) (end 149.425 106.61141) (width 0.25) (layer F.Cu) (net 6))
 (segment (start 149.425 106.61141) (end 148.63641 107.4) (width 0.25) (layer F.Cu) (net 6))
 (segment (start 148.63641 107.4) (end 148.43964 107.4) (width 0.25) (layer F.Cu) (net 6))
 (via (at 148.43964 107.4) (size 0.6) (drill 0.4) (layers F.Cu B.Cu) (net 6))
 (segment (start 149.7714 106.0036) (end 149.425 106.35) (width 0.25) (layer F.Cu) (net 6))
 (segment (start 150.0511 106.0036) (end 149.7714 106.0036) (width 0.25) (layer F.Cu) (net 6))
 (segment (start 150.45 108) (end 150.45 109.67) (width 0.25) (layer B.Cu) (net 7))
 (segment (start 150.45 109.67) (end 150.43 109.69) (width 0.25) (layer B.Cu) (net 7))
 (segment (start 150.175 106.2) (end 150.45 106.475) (width 0.25) (layer B.Cu) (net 8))
 (segment (start 150.45 106.475) (end 150.45 107.3) (width 0.25) (layer B.Cu) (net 8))
 (segment (start 147.8 106.2) (end 150.175 106.2) (width 0.25) (layer B.Cu) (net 8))
 (segment (start 146.9511 106.0036) (end 147.6036 106.0036) (width 0.25) (layer F.Cu) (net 8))
 (segment (start 147.6036 106.0036) (end 147.8 106.2) (width 0.25) (layer F.Cu) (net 8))
 (via (at 147.8 106.2) (size 0.6) (drill 0.4) (layers F.Cu B.Cu) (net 8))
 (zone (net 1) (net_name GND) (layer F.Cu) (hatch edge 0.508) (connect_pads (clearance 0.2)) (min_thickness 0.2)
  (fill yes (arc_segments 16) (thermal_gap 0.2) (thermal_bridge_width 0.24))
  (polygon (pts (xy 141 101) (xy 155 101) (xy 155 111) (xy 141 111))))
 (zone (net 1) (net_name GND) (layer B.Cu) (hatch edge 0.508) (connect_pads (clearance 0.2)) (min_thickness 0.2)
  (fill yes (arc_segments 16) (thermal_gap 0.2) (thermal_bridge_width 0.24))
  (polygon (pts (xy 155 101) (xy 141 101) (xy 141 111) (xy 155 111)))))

